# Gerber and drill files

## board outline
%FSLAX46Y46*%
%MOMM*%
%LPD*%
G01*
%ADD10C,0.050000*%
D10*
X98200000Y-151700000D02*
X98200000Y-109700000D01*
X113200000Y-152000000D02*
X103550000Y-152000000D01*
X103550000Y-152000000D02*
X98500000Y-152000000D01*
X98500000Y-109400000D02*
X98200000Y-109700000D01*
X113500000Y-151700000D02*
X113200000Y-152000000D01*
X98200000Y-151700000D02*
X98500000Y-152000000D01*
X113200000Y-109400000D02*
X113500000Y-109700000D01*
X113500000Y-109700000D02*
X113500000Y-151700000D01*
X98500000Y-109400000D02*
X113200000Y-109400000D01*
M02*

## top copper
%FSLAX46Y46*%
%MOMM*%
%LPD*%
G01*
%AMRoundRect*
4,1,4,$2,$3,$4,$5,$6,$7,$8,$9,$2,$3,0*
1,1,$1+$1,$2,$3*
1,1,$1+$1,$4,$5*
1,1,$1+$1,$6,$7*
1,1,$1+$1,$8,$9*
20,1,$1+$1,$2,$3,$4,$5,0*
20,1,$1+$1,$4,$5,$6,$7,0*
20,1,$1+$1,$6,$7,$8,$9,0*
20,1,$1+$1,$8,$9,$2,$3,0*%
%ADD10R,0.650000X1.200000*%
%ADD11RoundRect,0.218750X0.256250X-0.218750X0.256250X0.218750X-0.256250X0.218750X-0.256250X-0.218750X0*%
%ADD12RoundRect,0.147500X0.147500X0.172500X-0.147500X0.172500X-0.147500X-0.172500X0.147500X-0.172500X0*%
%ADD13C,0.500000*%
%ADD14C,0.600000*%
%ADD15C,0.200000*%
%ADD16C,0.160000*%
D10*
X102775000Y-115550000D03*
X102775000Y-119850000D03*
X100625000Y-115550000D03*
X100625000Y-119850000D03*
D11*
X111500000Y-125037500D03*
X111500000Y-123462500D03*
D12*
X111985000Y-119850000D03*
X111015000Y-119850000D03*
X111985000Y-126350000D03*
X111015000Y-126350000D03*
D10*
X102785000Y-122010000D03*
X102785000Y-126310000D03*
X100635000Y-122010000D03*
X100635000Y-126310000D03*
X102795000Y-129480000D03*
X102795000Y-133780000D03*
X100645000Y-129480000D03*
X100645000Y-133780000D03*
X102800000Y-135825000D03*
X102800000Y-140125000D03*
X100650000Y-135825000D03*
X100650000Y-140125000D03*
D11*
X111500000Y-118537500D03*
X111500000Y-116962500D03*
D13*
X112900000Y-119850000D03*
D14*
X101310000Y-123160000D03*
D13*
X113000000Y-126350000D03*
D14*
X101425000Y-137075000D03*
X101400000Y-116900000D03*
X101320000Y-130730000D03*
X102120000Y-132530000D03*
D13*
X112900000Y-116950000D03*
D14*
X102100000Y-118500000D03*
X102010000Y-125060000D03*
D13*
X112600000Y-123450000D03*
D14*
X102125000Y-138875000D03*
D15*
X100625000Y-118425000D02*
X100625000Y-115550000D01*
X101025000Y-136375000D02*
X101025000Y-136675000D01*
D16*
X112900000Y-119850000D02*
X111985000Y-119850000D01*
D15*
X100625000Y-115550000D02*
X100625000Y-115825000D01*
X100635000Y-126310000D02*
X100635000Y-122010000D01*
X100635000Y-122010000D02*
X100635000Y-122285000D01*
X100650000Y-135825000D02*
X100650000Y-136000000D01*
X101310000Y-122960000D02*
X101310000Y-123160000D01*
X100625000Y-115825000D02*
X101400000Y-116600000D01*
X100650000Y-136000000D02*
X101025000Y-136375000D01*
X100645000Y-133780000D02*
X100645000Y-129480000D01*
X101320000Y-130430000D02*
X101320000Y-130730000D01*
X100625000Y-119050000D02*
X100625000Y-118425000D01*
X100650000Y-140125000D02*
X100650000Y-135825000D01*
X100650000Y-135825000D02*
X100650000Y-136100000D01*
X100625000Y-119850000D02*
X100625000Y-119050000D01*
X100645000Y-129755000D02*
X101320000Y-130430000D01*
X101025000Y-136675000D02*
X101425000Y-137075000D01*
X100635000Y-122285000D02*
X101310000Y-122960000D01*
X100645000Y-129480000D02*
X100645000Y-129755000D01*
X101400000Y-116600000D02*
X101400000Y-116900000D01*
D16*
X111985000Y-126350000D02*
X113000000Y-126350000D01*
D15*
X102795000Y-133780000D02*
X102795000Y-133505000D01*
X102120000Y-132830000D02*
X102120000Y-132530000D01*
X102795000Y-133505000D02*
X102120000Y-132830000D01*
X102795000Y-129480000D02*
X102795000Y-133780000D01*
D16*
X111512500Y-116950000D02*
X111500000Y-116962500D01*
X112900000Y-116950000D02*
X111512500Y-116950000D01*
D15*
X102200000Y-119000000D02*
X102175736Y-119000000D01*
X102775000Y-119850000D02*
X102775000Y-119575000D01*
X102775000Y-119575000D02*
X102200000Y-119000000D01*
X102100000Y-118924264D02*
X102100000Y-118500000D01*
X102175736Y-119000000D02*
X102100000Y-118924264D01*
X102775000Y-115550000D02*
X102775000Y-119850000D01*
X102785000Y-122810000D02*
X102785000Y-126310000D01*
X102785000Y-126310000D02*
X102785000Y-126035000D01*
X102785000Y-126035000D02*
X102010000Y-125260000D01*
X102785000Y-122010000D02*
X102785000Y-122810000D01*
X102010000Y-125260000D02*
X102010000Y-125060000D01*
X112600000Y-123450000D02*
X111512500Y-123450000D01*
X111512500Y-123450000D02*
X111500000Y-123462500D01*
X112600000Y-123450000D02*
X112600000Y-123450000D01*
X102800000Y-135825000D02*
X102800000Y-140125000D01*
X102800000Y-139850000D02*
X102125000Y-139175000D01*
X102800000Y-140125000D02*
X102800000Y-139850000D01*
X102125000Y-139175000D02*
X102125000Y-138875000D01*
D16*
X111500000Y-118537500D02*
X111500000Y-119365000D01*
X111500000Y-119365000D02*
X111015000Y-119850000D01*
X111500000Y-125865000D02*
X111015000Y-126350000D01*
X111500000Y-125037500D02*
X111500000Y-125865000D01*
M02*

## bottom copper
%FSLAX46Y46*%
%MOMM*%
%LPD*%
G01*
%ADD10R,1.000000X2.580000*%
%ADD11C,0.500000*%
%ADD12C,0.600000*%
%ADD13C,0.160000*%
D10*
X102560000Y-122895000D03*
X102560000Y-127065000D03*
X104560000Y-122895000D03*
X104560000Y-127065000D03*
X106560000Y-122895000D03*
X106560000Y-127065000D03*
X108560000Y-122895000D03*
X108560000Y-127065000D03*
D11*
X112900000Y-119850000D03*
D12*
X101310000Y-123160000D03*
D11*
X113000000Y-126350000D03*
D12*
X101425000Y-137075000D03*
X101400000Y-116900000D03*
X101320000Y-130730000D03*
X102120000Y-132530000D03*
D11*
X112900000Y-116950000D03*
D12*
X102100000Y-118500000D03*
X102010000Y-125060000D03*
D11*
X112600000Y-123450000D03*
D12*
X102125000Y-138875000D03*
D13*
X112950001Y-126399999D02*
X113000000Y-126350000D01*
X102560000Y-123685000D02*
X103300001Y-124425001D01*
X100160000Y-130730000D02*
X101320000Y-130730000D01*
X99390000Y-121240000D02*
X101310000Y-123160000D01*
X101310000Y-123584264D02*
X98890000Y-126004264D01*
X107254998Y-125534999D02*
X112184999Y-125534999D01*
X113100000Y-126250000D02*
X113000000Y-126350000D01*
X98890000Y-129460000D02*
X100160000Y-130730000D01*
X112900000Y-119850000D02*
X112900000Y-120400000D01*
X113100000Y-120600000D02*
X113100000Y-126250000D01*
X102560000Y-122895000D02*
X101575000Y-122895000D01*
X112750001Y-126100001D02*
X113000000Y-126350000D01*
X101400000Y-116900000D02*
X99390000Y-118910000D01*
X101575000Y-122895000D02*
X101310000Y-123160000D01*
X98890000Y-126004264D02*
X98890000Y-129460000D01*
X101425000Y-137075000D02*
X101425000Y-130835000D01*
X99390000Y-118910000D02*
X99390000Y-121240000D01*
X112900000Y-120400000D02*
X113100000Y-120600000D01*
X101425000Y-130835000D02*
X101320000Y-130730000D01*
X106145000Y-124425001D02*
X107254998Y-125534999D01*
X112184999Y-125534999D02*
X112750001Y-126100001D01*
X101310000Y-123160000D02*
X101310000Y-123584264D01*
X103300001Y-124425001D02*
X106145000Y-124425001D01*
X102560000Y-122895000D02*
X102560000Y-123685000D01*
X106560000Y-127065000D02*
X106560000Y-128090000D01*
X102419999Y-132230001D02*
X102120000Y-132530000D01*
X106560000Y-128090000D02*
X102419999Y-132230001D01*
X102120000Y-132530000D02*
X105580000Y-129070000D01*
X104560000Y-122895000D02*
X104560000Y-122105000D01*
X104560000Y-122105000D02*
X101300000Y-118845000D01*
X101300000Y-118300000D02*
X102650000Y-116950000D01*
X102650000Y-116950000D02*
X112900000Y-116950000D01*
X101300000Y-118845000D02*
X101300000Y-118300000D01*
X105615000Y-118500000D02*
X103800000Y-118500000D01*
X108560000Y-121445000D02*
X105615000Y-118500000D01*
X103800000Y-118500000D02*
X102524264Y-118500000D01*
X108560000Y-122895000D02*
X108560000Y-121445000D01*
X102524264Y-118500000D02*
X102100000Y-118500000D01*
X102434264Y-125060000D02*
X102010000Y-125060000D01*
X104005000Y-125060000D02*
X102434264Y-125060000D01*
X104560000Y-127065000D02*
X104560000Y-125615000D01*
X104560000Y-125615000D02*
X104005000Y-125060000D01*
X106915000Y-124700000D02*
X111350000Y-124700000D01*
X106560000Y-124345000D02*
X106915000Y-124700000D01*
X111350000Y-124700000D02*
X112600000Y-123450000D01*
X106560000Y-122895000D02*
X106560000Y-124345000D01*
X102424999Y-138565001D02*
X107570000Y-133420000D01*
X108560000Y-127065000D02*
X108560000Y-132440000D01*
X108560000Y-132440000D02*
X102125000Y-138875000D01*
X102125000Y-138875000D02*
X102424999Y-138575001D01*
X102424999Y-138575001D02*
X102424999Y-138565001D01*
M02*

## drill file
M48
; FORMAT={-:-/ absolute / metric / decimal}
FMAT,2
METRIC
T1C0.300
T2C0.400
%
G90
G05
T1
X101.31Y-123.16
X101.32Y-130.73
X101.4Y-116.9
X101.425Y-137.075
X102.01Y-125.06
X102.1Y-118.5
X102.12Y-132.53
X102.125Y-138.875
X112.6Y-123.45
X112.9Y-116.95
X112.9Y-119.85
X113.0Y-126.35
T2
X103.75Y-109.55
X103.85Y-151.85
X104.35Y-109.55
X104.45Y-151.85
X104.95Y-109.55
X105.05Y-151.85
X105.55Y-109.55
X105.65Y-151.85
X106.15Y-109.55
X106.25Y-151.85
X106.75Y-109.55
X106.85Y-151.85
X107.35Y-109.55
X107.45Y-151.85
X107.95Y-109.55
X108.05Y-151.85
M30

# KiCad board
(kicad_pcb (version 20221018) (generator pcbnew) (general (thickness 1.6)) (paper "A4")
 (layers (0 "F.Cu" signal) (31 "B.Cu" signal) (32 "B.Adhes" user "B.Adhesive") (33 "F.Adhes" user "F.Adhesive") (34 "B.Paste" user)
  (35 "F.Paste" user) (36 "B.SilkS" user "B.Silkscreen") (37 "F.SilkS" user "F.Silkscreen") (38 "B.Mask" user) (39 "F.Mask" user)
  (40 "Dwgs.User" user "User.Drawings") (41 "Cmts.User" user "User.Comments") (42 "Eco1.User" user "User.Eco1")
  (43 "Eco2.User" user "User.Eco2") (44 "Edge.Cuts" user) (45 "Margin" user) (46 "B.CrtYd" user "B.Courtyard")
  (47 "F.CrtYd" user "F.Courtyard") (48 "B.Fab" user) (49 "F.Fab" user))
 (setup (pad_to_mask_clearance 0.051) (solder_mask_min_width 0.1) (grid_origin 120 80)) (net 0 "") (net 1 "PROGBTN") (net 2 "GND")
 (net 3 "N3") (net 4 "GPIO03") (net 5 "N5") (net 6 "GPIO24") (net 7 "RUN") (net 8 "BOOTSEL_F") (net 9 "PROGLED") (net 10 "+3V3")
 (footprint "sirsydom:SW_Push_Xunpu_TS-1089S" (layer "F.Cu") (at 101.7 117.7 -90)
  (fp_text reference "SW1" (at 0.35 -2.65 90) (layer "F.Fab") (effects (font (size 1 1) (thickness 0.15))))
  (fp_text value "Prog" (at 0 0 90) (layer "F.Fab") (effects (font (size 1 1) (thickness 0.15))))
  (pad "1" smd rect (at -2.15 -1.075 270) (size 1.2 0.65) (layers "F.Cu" "F.Paste" "F.Mask") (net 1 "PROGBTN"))
  (pad "1" smd rect (at 2.15 -1.075 270) (size 1.2 0.65) (layers "F.Cu" "F.Paste" "F.Mask") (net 1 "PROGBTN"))
  (pad "2" smd rect (at -2.15 1.075 270) (size 1.2 0.65) (layers "F.Cu" "F.Paste" "F.Mask") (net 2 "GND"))
  (pad "2" smd rect (at 2.15 1.075 270) (size 1.2 0.65) (layers "F.Cu" "F.Paste" "F.Mask") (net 2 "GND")))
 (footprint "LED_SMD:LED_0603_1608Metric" (layer "F.Cu") (at 111.5 124.25 90)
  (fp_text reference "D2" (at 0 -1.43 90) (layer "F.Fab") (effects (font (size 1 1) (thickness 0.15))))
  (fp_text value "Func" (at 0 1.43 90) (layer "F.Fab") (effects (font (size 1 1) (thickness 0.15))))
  (pad "1" smd roundrect (at -0.7875 0 90) (size 0.875 0.95) (layers "F.Cu" "F.Paste" "F.Mask") (roundrect_rratio 0.25) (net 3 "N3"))
  (pad "2" smd roundrect (at 0.7875 0 90) (size 0.875 0.95) (layers "F.Cu" "F.Paste" "F.Mask") (roundrect_rratio 0.25) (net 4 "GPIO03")))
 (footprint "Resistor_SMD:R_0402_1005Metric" (layer "F.Cu") (at 111.5 119.85 180)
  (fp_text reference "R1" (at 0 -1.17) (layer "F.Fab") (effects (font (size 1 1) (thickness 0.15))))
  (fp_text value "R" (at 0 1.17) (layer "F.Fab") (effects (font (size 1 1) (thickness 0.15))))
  (pad "1" smd roundrect (at -0.485 0 180) (size 0.59 0.64) (layers "F.Cu" "F.Paste" "F.Mask") (roundrect_rratio 0.25) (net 2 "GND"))
  (pad "2" smd roundrect (at 0.485 0 180) (size 0.59 0.64) (layers "F.Cu" "F.Paste" "F.Mask") (roundrect_rratio 0.25) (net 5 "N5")))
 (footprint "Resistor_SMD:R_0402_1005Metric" (layer "F.Cu") (at 111.5 126.35 180)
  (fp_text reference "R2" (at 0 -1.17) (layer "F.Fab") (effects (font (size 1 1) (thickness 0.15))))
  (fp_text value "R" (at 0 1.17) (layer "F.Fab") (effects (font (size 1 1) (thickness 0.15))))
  (pad "1" smd roundrect (at -0.485 0 180) (size 0.59 0.64) (layers "F.Cu" "F.Paste" "F.Mask") (roundrect_rratio 0.25) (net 2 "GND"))
  (pad "2" smd roundrect (at 0.485 0 180) (size 0.59 0.64) (layers "F.Cu" "F.Paste" "F.Mask") (roundrect_rratio 0.25) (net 3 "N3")))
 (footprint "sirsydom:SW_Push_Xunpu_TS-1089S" (layer "F.Cu") (at 101.71 124.16 -90)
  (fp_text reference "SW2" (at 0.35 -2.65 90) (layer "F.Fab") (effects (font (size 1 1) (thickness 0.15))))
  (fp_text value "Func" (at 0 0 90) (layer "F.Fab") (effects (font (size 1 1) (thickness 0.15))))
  (pad "1" smd rect (at -2.15 -1.075 270) (size 1.2 0.65) (layers "F.Cu" "F.Paste" "F.Mask") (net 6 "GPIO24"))
  (pad "1" smd rect (at 2.15 -1.075 270) (size 1.2 0.65) (layers "F.Cu" "F.Paste" "F.Mask") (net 6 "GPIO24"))
  (pad "2" smd rect (at -2.15 1.075 270) (size 1.2 0.65) (layers "F.Cu" "F.Paste" "F.Mask") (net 2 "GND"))
  (pad "2" smd rect (at 2.15 1.075 270) (size 1.2 0.65) (layers "F.Cu" "F.Paste" "F.Mask") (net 2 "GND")))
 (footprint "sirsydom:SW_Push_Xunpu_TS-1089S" (layer "F.Cu") (at 101.72 131.63 -90)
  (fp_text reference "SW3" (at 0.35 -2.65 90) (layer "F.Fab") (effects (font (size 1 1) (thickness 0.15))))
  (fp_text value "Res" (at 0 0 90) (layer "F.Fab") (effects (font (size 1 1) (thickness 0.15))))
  (pad "1" smd rect (at -2.15 -1.075 270) (size 1.2 0.65) (layers "F.Cu" "F.Paste" "F.Mask") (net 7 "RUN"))
  (pad "1" smd rect (at 2.15 -1.075 270) (size 1.2 0.65) (layers "F.Cu" "F.Paste" "F.Mask") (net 7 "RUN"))
  (pad "2" smd rect (at -2.15 1.075 270) (size 1.2 0.65) (layers "F.Cu" "F.Paste" "F.Mask") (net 2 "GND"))
  (pad "2" smd rect (at 2.15 1.075 270) (size 1.2 0.65) (layers "F.Cu" "F.Paste" "F.Mask") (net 2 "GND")))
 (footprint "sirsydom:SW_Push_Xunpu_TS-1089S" (layer "F.Cu") (at 101.725 137.975 -90)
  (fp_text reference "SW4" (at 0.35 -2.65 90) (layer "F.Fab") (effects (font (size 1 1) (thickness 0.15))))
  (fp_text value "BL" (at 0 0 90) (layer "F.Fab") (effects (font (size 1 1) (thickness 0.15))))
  (pad "1" smd rect (at -2.15 -1.075 270) (size 1.2 0.65) (layers "F.Cu" "F.Paste" "F.Mask") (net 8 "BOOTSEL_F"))
  (pad "1" smd rect (at 2.15 -1.075 270) (size 1.2 0.65) (layers "F.Cu" "F.Paste" "F.Mask") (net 8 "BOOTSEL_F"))
  (pad "2" smd rect (at -2.15 1.075 270) (size 1.2 0.65) (layers "F.Cu" "F.Paste" "F.Mask") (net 2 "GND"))
  (pad "2" smd rect (at 2.15 1.075 270) (size 1.2 0.65) (layers "F.Cu" "F.Paste" "F.Mask") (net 2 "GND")))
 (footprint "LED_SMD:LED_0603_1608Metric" (layer "F.Cu") (at 111.5 117.75 90)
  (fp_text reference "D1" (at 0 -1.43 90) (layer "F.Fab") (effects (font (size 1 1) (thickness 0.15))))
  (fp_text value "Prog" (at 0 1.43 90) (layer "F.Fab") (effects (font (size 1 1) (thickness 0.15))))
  (pad "1" smd roundrect (at -0.7875 0 90) (size 0.875 0.95) (layers "F.Cu" "F.Paste" "F.Mask") (roundrect_rratio 0.25) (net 5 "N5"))
  (pad "2" smd roundrect (at 0.7875 0 90) (size 0.875 0.95) (layers "F.Cu" "F.Paste" "F.Mask") (roundrect_rratio 0.25) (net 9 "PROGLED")))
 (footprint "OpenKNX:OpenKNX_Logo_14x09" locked (layer "F.Cu") (at 105.8 146.4)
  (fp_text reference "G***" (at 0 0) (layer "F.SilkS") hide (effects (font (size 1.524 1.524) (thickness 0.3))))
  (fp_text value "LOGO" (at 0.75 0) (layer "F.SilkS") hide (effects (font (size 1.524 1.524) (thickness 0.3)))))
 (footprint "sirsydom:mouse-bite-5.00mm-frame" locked (layer "F.Cu") (at 105.35 109.55)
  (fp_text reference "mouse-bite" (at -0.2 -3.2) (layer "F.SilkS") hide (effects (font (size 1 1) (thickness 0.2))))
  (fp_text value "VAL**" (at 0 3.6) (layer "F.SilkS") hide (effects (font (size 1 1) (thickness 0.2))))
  (pad "" np_thru_hole circle locked (at -1.6 0) (size 0.4 0.4) (drill 0.4) (layers "*.Cu" "*.Mask"))
  (pad "" np_thru_hole circle locked (at -1 0) (size 0.4 0.4) (drill 0.4) (layers "*.Cu" "*.Mask"))
  (pad "" np_thru_hole circle locked (at -0.4 0) (size 0.4 0.4) (drill 0.4) (layers "*.Cu" "*.Mask"))
  (pad "" np_thru_hole circle locked (at 0.2 0) (size 0.4 0.4) (drill 0.4) (layers "*.Cu" "*.Mask"))
  (pad "" np_thru_hole circle locked (at 0.8 0) (size 0.4 0.4) (drill 0.4) (layers "*.Cu" "*.Mask"))
  (pad "" np_thru_hole circle locked (at 1.4 0) (size 0.4 0.4) (drill 0.4) (layers "*.Cu" "*.Mask"))
  (pad "" np_thru_hole circle locked (at 2 0) (size 0.4 0.4) (drill 0.4) (layers "*.Cu" "*.Mask"))
  (pad "" np_thru_hole circle locked (at 2.6 0) (size 0.4 0.4) (drill 0.4) (layers "*.Cu" "*.Mask")))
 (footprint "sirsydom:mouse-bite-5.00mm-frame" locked (layer "F.Cu") (at 106.45 151.85 180)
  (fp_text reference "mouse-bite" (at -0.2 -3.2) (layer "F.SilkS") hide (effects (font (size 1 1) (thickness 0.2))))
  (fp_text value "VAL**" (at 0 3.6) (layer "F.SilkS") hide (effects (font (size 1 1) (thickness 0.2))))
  (pad "" np_thru_hole circle locked (at -1.6 0 180) (size 0.4 0.4) (drill 0.4) (layers "*.Cu" "*.Mask"))
  (pad "" np_thru_hole circle locked (at -1 0 180) (size 0.4 0.4) (drill 0.4) (layers "*.Cu" "*.Mask"))
  (pad "" np_thru_hole circle locked (at -0.4 0 180) (size 0.4 0.4) (drill 0.4) (layers "*.Cu" "*.Mask"))
  (pad "" np_thru_hole circle locked (at 0.2 0 180) (size 0.4 0.4) (drill 0.4) (layers "*.Cu" "*.Mask"))
  (pad "" np_thru_hole circle locked (at 0.8 0 180) (size 0.4 0.4) (drill 0.4) (layers "*.Cu" "*.Mask"))
  (pad "" np_thru_hole circle locked (at 1.4 0 180) (size 0.4 0.4) (drill 0.4) (layers "*.Cu" "*.Mask"))
  (pad "" np_thru_hole circle locked (at 2 0 180) (size 0.4 0.4) (drill 0.4) (layers "*.Cu" "*.Mask"))
  (pad "" np_thru_hole circle locked (at 2.6 0 180) (size 0.4 0.4) (drill 0.4) (layers "*.Cu" "*.Mask")))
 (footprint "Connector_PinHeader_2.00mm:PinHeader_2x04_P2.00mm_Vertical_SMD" (layer "B.Cu") (at 105.56 124.98 -90)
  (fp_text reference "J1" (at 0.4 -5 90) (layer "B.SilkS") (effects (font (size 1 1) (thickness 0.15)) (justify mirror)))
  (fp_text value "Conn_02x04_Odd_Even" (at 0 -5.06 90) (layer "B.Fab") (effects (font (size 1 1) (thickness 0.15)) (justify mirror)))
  (pad "1" smd rect (at -2.085 3 270) (size 2.58 1) (layers "B.Cu" "B.Paste" "B.Mask") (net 2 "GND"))
  (pad "2" smd rect (at 2.085 3 270) (size 2.58 1) (layers "B.Cu" "B.Paste" "B.Mask") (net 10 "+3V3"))
  (pad "3" smd rect (at -2.085 1 270) (size 2.58 1) (layers "B.Cu" "B.Paste" "B.Mask") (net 9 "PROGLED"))
  (pad "4" smd rect (at 2.085 1 270) (size 2.58 1) (layers "B.Cu" "B.Paste" "B.Mask") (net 6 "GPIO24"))
  (pad "5" smd rect (at -2.085 -1 270) (size 2.58 1) (layers "B.Cu" "B.Paste" "B.Mask") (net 4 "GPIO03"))
  (pad "6" smd rect (at 2.085 -1 270) (size 2.58 1) (layers "B.Cu" "B.Paste" "B.Mask") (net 7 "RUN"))
  (pad "7" smd rect (at -2.085 -3 270) (size 2.58 1) (layers "B.Cu" "B.Paste" "B.Mask") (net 1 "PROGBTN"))
  (pad "8" smd rect (at 2.085 -3 270) (size 2.58 1) (layers "B.Cu" "B.Paste" "B.Mask") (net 8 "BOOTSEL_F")))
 (gr_line (start 98.2 151.7) (end 98.2 109.7) (stroke (width 0.05) (type solid)) (layer "Edge.Cuts"))
 (gr_line (start 113.2 152) (end 103.55 152) (stroke (width 0.05) (type solid)) (layer "Edge.Cuts"))
 (gr_line (start 103.55 152) (end 98.5 152) (stroke (width 0.05) (type solid)) (layer "Edge.Cuts"))
 (gr_line (start 98.5 109.4) (end 98.2 109.7) (stroke (width 0.05) (type solid)) (layer "Edge.Cuts"))
 (gr_line (start 113.5 151.7) (end 113.2 152) (stroke (width 0.05) (type solid)) (layer "Edge.Cuts"))
 (gr_line (start 98.2 151.7) (end 98.5 152) (stroke (width 0.05) (type solid)) (layer "Edge.Cuts"))
 (gr_line (start 113.2 109.4) (end 113.5 109.7) (stroke (width 0.05) (type solid)) (layer "Edge.Cuts"))
 (gr_line (start 113.5 109.7) (end 113.5 151.7) (stroke (width 0.05) (type solid)) (layer "Edge.Cuts"))
 (gr_line (start 98.5 109.4) (end 113.2 109.4) (stroke (width 0.05) (type solid)) (layer "Edge.Cuts"))
 (segment (start 100.625 118.425) (end 100.625 115.55) (width 0.2) (layer "F.Cu") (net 2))
 (segment (start 101.025 136.375) (end 101.025 136.675) (width 0.2) (layer "F.Cu") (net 2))
 (segment (start 112.9 119.85) (end 111.985 119.85) (width 0.16) (layer "F.Cu") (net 2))
 (segment (start 100.625 115.55) (end 100.625 115.825) (width 0.2) (layer "F.Cu") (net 2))
 (segment (start 100.635 126.31) (end 100.635 122.01) (width 0.2) (layer "F.Cu") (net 2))
 (segment (start 100.635 122.01) (end 100.635 122.285) (width 0.2) (layer "F.Cu") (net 2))
 (segment (start 100.65 135.825) (end 100.65 136) (width 0.2) (layer "F.Cu") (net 2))
 (segment (start 101.31 122.96) (end 101.31 123.16) (width 0.2) (layer "F.Cu") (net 2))
 (segment (start 100.625 115.825) (end 101.4 116.6) (width 0.2) (layer "F.Cu") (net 2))
 (segment (start 100.65 136) (end 101.025 136.375) (width 0.2) (layer "F.Cu") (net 2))
 (segment (start 100.645 133.78) (end 100.645 129.48) (width 0.2) (layer "F.Cu") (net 2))
 (segment (start 101.32 130.43) (end 101.32 130.73) (width 0.2) (layer "F.Cu") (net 2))
 (segment (start 100.625 119.05) (end 100.625 118.425) (width 0.2) (layer "F.Cu") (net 2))
 (segment (start 100.65 140.125) (end 100.65 135.825) (width 0.2) (layer "F.Cu") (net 2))
 (segment (start 100.65 135.825) (end 100.65 136.1) (width 0.2) (layer "F.Cu") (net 2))
 (segment (start 100.625 119.85) (end 100.625 119.05) (width 0.2) (layer "F.Cu") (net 2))
 (segment (start 100.645 129.755) (end 101.32 130.43) (width 0.2) (layer "F.Cu") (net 2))
 (segment (start 101.025 136.675) (end 101.425 137.075) (width 0.2) (layer "F.Cu") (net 2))
 (segment (start 100.635 122.285) (end 101.31 122.96) (width 0.2) (layer "F.Cu") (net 2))
 (segment (start 100.645 129.48) (end 100.645 129.755) (width 0.2) (layer "F.Cu") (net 2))
 (segment (start 101.4 116.6) (end 101.4 116.9) (width 0.2) (layer "F.Cu") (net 2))
 (segment (start 111.985 126.35) (end 113 126.35) (width 0.16) (layer "F.Cu") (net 2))
 (via (at 112.9 119.85) (size 0.5) (drill 0.3) (layers "F.Cu" "B.Cu") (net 2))
 (via (at 101.31 123.16) (size 0.6) (drill 0.3) (layers "F.Cu" "B.Cu") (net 2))
 (via (at 113 126.35) (size 0.5) (drill 0.3) (layers "F.Cu" "B.Cu") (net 2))
 (via (at 101.425 137.075) (size 0.6) (drill 0.3) (layers "F.Cu" "B.Cu") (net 2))
 (via (at 101.4 116.9) (size 0.6) (drill 0.3) (layers "F.Cu" "B.Cu") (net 2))
 (via (at 101.32 130.73) (size 0.6) (drill 0.3) (layers "F.Cu" "B.Cu") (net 2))
 (segment (start 112.950001 126.399999) (end 113 126.35) (width 0.16) (layer "B.Cu") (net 2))
 (segment (start 102.56 123.685) (end 103.300001 124.425001) (width 0.16) (layer "B.Cu") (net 2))
 (segment (start 100.16 130.73) (end 101.32 130.73) (width 0.16) (layer "B.Cu") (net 2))
 (segment (start 99.39 121.24) (end 101.31 123.16) (width 0.16) (layer "B.Cu") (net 2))
 (segment (start 101.31 123.584264) (end 98.89 126.004264) (width 0.16) (layer "B.Cu") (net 2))
 (segment (start 107.254998 125.534999) (end 112.184999 125.534999) (width 0.16) (layer "B.Cu") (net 2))
 (segment (start 113.1 126.25) (end 113 126.35) (width 0.16) (layer "B.Cu") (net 2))
 (segment (start 98.89 129.46) (end 100.16 130.73) (width 0.16) (layer "B.Cu") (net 2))
 (segment (start 112.9 119.85) (end 112.9 120.4) (width 0.16) (layer "B.Cu") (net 2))
 (segment (start 113.1 120.6) (end 113.1 126.25) (width 0.16) (layer "B.Cu") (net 2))
 (segment (start 102.56 122.895) (end 101.575 122.895) (width 0.16) (layer "B.Cu") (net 2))
 (segment (start 112.750001 126.100001) (end 113 126.35) (width 0.16) (layer "B.Cu") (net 2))
 (segment (start 101.4 116.9) (end 99.39 118.91) (width 0.16) (layer "B.Cu") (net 2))
 (segment (start 101.575 122.895) (end 101.31 123.16) (width 0.16) (layer "B.Cu") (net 2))
 (segment (start 98.89 126.004264) (end 98.89 129.46) (width 0.16) (layer "B.Cu") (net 2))
 (segment (start 101.425 137.075) (end 101.425 130.835) (width 0.16) (layer "B.Cu") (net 2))
 (segment (start 99.39 118.91) (end 99.39 121.24) (width 0.16) (layer "B.Cu") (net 2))
 (segment (start 112.9 120.4) (end 113.1 120.6) (width 0.16) (layer "B.Cu") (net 2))
 (segment (start 101.425 130.835) (end 101.32 130.73) (width 0.16) (layer "B.Cu") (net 2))
 (segment (start 106.145 124.425001) (end 107.254998 125.534999) (width 0.16) (layer "B.Cu") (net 2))
 (segment (start 112.184999 125.534999) (end 112.750001 126.100001) (width 0.16) (layer "B.Cu") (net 2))
 (segment (start 101.31 123.16) (end 101.31 123.584264) (width 0.16) (layer "B.Cu") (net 2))
 (segment (start 103.300001 124.425001) (end 106.145 124.425001) (width 0.16) (layer "B.Cu") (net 2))
 (segment (start 102.56 122.895) (end 102.56 123.685) (width 0.16) (layer "B.Cu") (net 2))
 (segment (start 102.795 133.78) (end 102.795 133.505) (width 0.2) (layer "F.Cu") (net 7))
 (segment (start 102.12 132.83) (end 102.12 132.53) (width 0.2) (layer "F.Cu") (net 7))
 (segment (start 102.795 133.505) (end 102.12 132.83) (width 0.2) (layer "F.Cu") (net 7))
 (segment (start 102.795 129.48) (end 102.795 133.78) (width 0.2) (layer "F.Cu") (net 7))
 (via (at 102.12 132.53) (size 0.6) (drill 0.3) (layers "F.Cu" "B.Cu") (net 7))
 (segment (start 106.56 127.065) (end 106.56 128.09) (width 0.16) (layer "B.Cu") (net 7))
 (segment (start 102.419999 132.230001) (end 102.12 132.53) (width 0.16) (layer "B.Cu") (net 7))
 (segment (start 106.56 128.09) (end 102.419999 132.230001) (width 0.16) (layer "B.Cu") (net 7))
 (segment (start 102.12 132.53) (end 105.58 129.07) (width 0.16) (layer "B.Cu") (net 7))
 (segment (start 111.5125 116.95) (end 111.5 116.9625) (width 0.16) (layer "F.Cu") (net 9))
 (segment (start 112.9 116.95) (end 111.5125 116.95) (width 0.16) (layer "F.Cu") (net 9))
 (via (at 112.9 116.95) (size 0.5) (drill 0.3) (layers "F.Cu" "B.Cu") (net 9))
 (segment (start 104.56 122.895) (end 104.56 122.105) (width 0.16) (layer "B.Cu") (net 9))
 (segment (start 104.56 122.105) (end 101.3 118.845) (width 0.16) (layer "B.Cu") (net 9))
 (segment (start 101.3 118.3) (end 102.65 116.95) (width 0.16) (layer "B.Cu") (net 9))
 (segment (start 102.65 116.95) (end 112.9 116.95) (width 0.16) (layer "B.Cu") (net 9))
 (segment (start 101.3 118.845) (end 101.3 118.3) (width 0.16) (layer "B.Cu") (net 9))
 (segment (start 102.2 119) (end 102.175736 119) (width 0.2) (layer "F.Cu") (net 1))
 (segment (start 102.775 119.85) (end 102.775 119.575) (width 0.2) (layer "F.Cu") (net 1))
 (segment (start 102.775 119.575) (end 102.2 119) (width 0.2) (layer "F.Cu") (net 1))
 (segment (start 102.1 118.924264) (end 102.1 118.5) (width 0.2) (layer "F.Cu") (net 1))
 (segment (start 102.175736 119) (end 102.1 118.924264) (width 0.2) (layer "F.Cu") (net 1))
 (segment (start 102.775 115.55) (end 102.775 119.85) (width 0.2) (layer "F.Cu") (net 1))
 (via (at 102.1 118.5) (size 0.6) (drill 0.3) (layers "F.Cu" "B.Cu") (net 1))
 (segment (start 105.615 118.5) (end 103.8 118.5) (width 0.16) (layer "B.Cu") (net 1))
 (segment (start 108.56 121.445) (end 105.615 118.5) (width 0.16) (layer "B.Cu") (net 1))
 (segment (start 103.8 118.5) (end 102.524264 118.5) (width 0.16) (layer "B.Cu") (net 1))
 (segment (start 108.56 122.895) (end 108.56 121.445) (width 0.16) (layer "B.Cu") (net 1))
 (segment (start 102.524264 118.5) (end 102.1 118.5) (width 0.16) (layer "B.Cu") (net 1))
 (segment (start 102.785 122.81) (end 102.785 126.31) (width 0.2) (layer "F.Cu") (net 6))
 (segment (start 102.785 126.31) (end 102.785 126.035) (width 0.2) (layer "F.Cu") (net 6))
 (segment (start 102.785 126.035) (end 102.01 125.26) (width 0.2) (layer "F.Cu") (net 6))
 (segment (start 102.785 122.01) (end 102.785 122.81) (width 0.2) (layer "F.Cu") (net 6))
 (segment (start 102.01 125.26) (end 102.01 125.06) (width 0.2) (layer "F.Cu") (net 6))
 (via (at 102.01 125.06) (size 0.6) (drill 0.3) (layers "F.Cu" "B.Cu") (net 6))
 (segment (start 102.434264 125.06) (end 102.01 125.06) (width 0.16) (layer "B.Cu") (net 6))
 (segment (start 104.005 125.06) (end 102.434264 125.06) (width 0.16) (layer "B.Cu") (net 6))
 (segment (start 104.56 127.065) (end 104.56 125.615) (width 0.16) (layer "B.Cu") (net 6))
 (segment (start 104.56 125.615) (end 104.005 125.06) (width 0.16) (layer "B.Cu") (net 6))
 (segment (start 112.6 123.45) (end 111.5125 123.45) (width 0.2) (layer "F.Cu") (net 4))
 (segment (start 111.5125 123.45) (end 111.5 123.4625) (width 0.2) (layer "F.Cu") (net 4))
 (segment (start 112.6 123.45) (end 112.6 123.45) (width 0.2) (layer "F.Cu") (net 4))
 (via (at 112.6 123.45) (size 0.5) (drill 0.3) (layers "F.Cu" "B.Cu") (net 4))
 (segment (start 106.915 124.7) (end 111.35 124.7) (width 0.16) (layer "B.Cu") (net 4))
 (segment (start 106.56 124.345) (end 106.915 124.7) (width 0.16) (layer "B.Cu") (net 4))
 (segment (start 111.35 124.7) (end 112.6 123.45) (width 0.16) (layer "B.Cu") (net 4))
 (segment (start 106.56 122.895) (end 106.56 124.345) (width 0.16) (layer "B.Cu") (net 4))
 (segment (start 102.8 135.825) (end 102.8 140.125) (width 0.2) (layer "F.Cu") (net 8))
 (segment (start 102.8 139.85) (end 102.125 139.175) (width 0.2) (layer "F.Cu") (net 8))
 (segment (start 102.8 140.125) (end 102.8 139.85) (width 0.2) (layer "F.Cu") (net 8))
 (segment (start 102.125 139.175) (end 102.125 138.875) (width 0.2) (layer "F.Cu") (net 8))
 (via (at 102.125 138.875) (size 0.6) (drill 0.3) (layers "F.Cu" "B.Cu") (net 8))
 (segment (start 102.424999 138.565001) (end 107.57 133.42) (width 0.16) (layer "B.Cu") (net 8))
 (segment (start 108.56 127.065) (end 108.56 132.44) (width 0.16) (layer "B.Cu") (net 8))
 (segment (start 108.56 132.44) (end 102.125 138.875) (width 0.16) (layer "B.Cu") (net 8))
 (segment (start 102.125 138.875) (end 102.424999 138.575001) (width 0.16) (layer "B.Cu") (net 8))
 (segment (start 102.424999 138.575001) (end 102.424999 138.565001) (width 0.16) (layer "B.Cu") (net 8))
 (segment (start 111.5 118.5375) (end 111.5 119.365) (width 0.16) (layer "F.Cu") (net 5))
 (segment (start 111.5 119.365) (end 111.015 119.85) (width 0.16) (layer "F.Cu") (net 5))
 (segment (start 111.5 125.865) (end 111.015 126.35) (width 0.16) (layer "F.Cu") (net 3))
 (segment (start 111.5 125.0375) (end 111.5 125.865) (width 0.16) (layer "F.Cu") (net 3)))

